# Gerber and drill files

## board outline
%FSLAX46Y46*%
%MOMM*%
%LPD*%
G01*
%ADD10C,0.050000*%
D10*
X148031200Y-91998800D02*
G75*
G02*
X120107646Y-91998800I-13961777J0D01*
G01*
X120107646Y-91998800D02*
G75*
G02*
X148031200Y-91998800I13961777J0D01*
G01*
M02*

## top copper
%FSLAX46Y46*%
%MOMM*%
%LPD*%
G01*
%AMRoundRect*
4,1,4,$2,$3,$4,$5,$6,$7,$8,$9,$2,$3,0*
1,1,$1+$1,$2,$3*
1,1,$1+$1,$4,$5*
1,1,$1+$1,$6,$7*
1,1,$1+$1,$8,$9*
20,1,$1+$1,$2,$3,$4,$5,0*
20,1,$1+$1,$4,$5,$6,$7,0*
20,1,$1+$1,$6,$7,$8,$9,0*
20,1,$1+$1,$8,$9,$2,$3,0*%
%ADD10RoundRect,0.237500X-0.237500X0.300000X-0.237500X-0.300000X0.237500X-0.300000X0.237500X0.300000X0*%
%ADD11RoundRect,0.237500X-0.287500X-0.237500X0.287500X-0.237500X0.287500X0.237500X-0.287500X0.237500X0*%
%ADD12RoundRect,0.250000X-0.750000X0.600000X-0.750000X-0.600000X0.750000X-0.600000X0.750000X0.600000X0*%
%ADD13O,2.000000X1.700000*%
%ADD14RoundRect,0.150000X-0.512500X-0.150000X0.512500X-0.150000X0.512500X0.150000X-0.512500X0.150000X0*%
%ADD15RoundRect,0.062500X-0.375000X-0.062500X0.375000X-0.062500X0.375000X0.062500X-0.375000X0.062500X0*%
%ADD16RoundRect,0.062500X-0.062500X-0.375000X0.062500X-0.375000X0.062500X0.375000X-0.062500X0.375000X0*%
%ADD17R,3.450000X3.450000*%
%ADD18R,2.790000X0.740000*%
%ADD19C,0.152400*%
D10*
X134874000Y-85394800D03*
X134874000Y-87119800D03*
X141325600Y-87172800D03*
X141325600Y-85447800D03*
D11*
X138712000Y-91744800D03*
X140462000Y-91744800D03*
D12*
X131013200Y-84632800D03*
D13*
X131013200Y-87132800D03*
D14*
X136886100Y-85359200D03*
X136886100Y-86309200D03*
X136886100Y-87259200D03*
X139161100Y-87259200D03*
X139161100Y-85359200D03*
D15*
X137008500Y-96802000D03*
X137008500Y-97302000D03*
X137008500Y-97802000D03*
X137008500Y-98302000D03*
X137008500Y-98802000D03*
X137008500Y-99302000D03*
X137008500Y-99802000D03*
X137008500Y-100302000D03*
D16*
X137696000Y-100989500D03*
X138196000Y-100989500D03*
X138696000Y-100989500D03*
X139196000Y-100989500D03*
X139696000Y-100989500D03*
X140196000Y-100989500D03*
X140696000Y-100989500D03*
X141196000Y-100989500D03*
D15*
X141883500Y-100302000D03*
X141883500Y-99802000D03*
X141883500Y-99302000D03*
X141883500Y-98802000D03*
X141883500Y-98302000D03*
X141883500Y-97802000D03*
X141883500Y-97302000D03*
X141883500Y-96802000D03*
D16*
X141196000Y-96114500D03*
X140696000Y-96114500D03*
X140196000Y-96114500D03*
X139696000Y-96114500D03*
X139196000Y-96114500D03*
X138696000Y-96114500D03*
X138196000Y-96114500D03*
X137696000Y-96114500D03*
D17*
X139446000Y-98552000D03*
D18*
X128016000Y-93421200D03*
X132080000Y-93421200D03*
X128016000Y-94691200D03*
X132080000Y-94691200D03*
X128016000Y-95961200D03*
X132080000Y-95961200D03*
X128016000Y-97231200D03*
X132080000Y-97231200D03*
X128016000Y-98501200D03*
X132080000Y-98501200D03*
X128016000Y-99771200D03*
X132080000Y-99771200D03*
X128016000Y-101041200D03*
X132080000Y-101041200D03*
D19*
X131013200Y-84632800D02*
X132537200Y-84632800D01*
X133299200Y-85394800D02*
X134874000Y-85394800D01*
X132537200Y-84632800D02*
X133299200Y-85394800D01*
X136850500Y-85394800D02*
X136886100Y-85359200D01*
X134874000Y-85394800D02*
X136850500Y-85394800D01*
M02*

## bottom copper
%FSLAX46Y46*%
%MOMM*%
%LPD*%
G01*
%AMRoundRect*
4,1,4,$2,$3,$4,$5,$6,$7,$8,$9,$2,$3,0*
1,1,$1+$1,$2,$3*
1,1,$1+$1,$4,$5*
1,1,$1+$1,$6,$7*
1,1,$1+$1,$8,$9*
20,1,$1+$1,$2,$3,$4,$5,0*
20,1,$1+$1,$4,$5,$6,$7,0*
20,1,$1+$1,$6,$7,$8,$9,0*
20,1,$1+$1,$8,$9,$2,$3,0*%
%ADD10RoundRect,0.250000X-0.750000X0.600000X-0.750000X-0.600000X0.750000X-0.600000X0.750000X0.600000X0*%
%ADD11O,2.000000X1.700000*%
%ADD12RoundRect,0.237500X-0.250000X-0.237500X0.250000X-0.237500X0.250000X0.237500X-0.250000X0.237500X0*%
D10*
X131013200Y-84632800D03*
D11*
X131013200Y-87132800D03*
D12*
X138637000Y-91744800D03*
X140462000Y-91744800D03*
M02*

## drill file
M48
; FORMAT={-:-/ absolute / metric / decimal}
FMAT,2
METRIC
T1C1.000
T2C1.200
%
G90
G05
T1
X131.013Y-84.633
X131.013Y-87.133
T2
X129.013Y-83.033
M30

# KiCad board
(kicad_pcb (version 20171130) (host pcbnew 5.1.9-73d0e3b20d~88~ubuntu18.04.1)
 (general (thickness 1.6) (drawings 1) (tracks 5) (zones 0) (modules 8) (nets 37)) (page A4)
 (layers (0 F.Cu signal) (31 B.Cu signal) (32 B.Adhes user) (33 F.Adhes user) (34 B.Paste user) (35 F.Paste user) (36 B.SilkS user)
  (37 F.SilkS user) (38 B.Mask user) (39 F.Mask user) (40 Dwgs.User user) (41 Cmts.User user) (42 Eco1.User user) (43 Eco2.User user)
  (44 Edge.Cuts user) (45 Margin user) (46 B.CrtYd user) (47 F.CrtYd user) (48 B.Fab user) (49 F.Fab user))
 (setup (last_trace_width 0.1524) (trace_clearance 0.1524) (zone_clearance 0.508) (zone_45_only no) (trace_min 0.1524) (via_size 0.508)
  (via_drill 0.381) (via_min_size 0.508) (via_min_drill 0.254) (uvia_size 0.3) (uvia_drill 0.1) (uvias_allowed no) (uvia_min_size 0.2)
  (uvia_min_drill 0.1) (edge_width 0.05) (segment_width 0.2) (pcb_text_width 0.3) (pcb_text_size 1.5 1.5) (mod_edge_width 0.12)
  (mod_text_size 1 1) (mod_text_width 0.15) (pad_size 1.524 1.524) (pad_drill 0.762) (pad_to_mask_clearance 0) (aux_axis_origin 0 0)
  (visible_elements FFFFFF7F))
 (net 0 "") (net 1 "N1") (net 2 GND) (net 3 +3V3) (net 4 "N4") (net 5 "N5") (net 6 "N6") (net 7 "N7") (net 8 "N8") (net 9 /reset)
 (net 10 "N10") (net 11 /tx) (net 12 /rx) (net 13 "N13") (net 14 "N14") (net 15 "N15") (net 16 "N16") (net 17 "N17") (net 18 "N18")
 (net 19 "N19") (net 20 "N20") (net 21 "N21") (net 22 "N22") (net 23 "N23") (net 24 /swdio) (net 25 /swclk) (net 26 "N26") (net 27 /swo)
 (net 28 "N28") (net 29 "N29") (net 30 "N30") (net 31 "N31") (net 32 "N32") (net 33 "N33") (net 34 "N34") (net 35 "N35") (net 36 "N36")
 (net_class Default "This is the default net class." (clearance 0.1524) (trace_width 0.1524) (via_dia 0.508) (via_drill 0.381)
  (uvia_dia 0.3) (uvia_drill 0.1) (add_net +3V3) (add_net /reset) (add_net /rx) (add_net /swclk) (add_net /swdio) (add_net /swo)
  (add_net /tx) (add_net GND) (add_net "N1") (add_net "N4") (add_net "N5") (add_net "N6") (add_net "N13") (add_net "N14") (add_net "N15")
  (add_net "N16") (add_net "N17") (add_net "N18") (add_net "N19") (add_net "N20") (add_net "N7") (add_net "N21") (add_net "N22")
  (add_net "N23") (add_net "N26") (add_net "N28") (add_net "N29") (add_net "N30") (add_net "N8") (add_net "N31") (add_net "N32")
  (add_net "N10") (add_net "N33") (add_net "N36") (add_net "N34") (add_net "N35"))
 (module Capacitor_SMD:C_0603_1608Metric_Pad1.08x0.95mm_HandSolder (layer F.Cu) (at 134.874 86.2573 270)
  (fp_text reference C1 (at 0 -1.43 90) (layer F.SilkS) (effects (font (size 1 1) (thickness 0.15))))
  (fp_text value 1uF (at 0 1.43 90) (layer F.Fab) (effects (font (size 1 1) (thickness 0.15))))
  (pad 1 smd roundrect (at -0.8625 0 270) (size 1.075 0.95) (layers F.Cu F.Paste F.Mask) (roundrect_rratio 0.25) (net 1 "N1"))
  (pad 2 smd roundrect (at 0.8625 0 270) (size 1.075 0.95) (layers F.Cu F.Paste F.Mask) (roundrect_rratio 0.25) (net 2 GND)))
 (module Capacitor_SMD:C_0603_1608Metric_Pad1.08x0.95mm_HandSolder (layer F.Cu) (at 141.3256 86.3103 270)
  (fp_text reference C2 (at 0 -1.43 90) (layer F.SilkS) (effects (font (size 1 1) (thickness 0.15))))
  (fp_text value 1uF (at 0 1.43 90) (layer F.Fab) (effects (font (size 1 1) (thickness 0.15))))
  (pad 2 smd roundrect (at 0.8625 0 270) (size 1.075 0.95) (layers F.Cu F.Paste F.Mask) (roundrect_rratio 0.25) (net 2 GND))
  (pad 1 smd roundrect (at -0.8625 0 270) (size 1.075 0.95) (layers F.Cu F.Paste F.Mask) (roundrect_rratio 0.25) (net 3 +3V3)))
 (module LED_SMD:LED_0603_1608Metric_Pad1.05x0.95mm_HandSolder (layer F.Cu) (at 139.587 91.7448)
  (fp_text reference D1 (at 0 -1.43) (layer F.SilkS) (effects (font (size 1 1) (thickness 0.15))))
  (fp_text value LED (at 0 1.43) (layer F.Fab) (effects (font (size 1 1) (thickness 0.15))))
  (pad 1 smd roundrect (at -0.875 0) (size 1.05 0.95) (layers F.Cu F.Paste F.Mask) (roundrect_rratio 0.25) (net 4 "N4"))
  (pad 2 smd roundrect (at 0.875 0) (size 1.05 0.95) (layers F.Cu F.Paste F.Mask) (roundrect_rratio 0.25) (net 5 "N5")))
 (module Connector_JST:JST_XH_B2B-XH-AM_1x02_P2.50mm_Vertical (layer F.Cu) (at 131.0132 84.6328 270)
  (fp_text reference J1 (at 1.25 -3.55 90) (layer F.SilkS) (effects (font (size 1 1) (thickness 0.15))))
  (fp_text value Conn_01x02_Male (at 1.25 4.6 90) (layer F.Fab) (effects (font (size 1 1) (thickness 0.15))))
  (pad 1 thru_hole roundrect (at 0 0 270) (size 1.7 2) (drill 1) (layers *.Cu *.Mask) (roundrect_rratio 0.147059) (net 1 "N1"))
  (pad 2 thru_hole oval (at 2.5 0 270) (size 1.7 2) (drill 1) (layers *.Cu *.Mask) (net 2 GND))
  (pad "" np_thru_hole circle (at -1.6 2 270) (size 1.2 1.2) (drill 1.2) (layers *.Cu *.Mask)))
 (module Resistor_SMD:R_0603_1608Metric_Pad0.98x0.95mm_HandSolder (layer B.Cu) (at 139.5495 91.7448)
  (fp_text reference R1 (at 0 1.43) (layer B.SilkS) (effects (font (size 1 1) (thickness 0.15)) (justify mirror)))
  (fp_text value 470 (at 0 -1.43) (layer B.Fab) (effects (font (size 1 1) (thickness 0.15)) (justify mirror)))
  (pad 1 smd roundrect (at -0.9125 0) (size 0.975 0.95) (layers B.Cu B.Paste B.Mask) (roundrect_rratio 0.25) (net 3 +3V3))
  (pad 2 smd roundrect (at 0.9125 0) (size 0.975 0.95) (layers B.Cu B.Paste B.Mask) (roundrect_rratio 0.25) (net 5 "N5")))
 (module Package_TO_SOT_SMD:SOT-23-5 (layer F.Cu) (at 138.0236 86.3092)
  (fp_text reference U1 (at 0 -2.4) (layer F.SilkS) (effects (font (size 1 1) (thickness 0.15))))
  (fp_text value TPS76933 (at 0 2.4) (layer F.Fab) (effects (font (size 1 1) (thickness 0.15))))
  (pad 1 smd roundrect (at -1.1375 -0.95) (size 1.325 0.6) (layers F.Cu F.Paste F.Mask) (roundrect_rratio 0.25) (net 1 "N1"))
  (pad 2 smd roundrect (at -1.1375 0) (size 1.325 0.6) (layers F.Cu F.Paste F.Mask) (roundrect_rratio 0.25) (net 2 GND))
  (pad 3 smd roundrect (at -1.1375 0.95) (size 1.325 0.6) (layers F.Cu F.Paste F.Mask) (roundrect_rratio 0.25) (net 2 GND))
  (pad 4 smd roundrect (at 1.1375 0.95) (size 1.325 0.6) (layers F.Cu F.Paste F.Mask) (roundrect_rratio 0.25) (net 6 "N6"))
  (pad 5 smd roundrect (at 1.1375 -0.95) (size 1.325 0.6) (layers F.Cu F.Paste F.Mask) (roundrect_rratio 0.25) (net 3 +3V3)))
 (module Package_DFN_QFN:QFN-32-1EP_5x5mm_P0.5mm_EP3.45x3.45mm (layer F.Cu) (at 139.446 98.552)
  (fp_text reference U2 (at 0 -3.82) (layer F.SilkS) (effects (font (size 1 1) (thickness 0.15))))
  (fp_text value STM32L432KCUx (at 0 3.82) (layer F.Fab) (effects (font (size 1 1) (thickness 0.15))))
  (pad 1 smd roundrect (at -2.4375 -1.75) (size 0.875 0.25) (layers F.Cu F.Paste F.Mask) (roundrect_rratio 0.25) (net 3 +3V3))
  (pad 2 smd roundrect (at -2.4375 -1.25) (size 0.875 0.25) (layers F.Cu F.Paste F.Mask) (roundrect_rratio 0.25) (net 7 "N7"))
  (pad 3 smd roundrect (at -2.4375 -0.75) (size 0.875 0.25) (layers F.Cu F.Paste F.Mask) (roundrect_rratio 0.25) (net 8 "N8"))
  (pad 4 smd roundrect (at -2.4375 -0.25) (size 0.875 0.25) (layers F.Cu F.Paste F.Mask) (roundrect_rratio 0.25) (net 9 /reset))
  (pad 5 smd roundrect (at -2.4375 0.25) (size 0.875 0.25) (layers F.Cu F.Paste F.Mask) (roundrect_rratio 0.25) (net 3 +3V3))
  (pad 6 smd roundrect (at -2.4375 0.75) (size 0.875 0.25) (layers F.Cu F.Paste F.Mask) (roundrect_rratio 0.25) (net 4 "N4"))
  (pad 7 smd roundrect (at -2.4375 1.25) (size 0.875 0.25) (layers F.Cu F.Paste F.Mask) (roundrect_rratio 0.25) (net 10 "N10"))
  (pad 8 smd roundrect (at -2.4375 1.75) (size 0.875 0.25) (layers F.Cu F.Paste F.Mask) (roundrect_rratio 0.25) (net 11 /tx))
  (pad 9 smd roundrect (at -1.75 2.4375) (size 0.25 0.875) (layers F.Cu F.Paste F.Mask) (roundrect_rratio 0.25) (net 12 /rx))
  (pad 10 smd roundrect (at -1.25 2.4375) (size 0.25 0.875) (layers F.Cu F.Paste F.Mask) (roundrect_rratio 0.25) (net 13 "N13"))
  (pad 11 smd roundrect (at -0.75 2.4375) (size 0.25 0.875) (layers F.Cu F.Paste F.Mask) (roundrect_rratio 0.25) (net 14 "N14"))
  (pad 12 smd roundrect (at -0.25 2.4375) (size 0.25 0.875) (layers F.Cu F.Paste F.Mask) (roundrect_rratio 0.25) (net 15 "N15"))
  (pad 13 smd roundrect (at 0.25 2.4375) (size 0.25 0.875) (layers F.Cu F.Paste F.Mask) (roundrect_rratio 0.25) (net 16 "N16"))
  (pad 14 smd roundrect (at 0.75 2.4375) (size 0.25 0.875) (layers F.Cu F.Paste F.Mask) (roundrect_rratio 0.25) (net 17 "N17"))
  (pad 15 smd roundrect (at 1.25 2.4375) (size 0.25 0.875) (layers F.Cu F.Paste F.Mask) (roundrect_rratio 0.25) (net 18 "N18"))
  (pad 16 smd roundrect (at 1.75 2.4375) (size 0.25 0.875) (layers F.Cu F.Paste F.Mask) (roundrect_rratio 0.25) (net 2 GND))
  (pad 17 smd roundrect (at 2.4375 1.75) (size 0.875 0.25) (layers F.Cu F.Paste F.Mask) (roundrect_rratio 0.25) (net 3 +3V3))
  (pad 18 smd roundrect (at 2.4375 1.25) (size 0.875 0.25) (layers F.Cu F.Paste F.Mask) (roundrect_rratio 0.25) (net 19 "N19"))
  (pad 19 smd roundrect (at 2.4375 0.75) (size 0.875 0.25) (layers F.Cu F.Paste F.Mask) (roundrect_rratio 0.25) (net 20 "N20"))
  (pad 20 smd roundrect (at 2.4375 0.25) (size 0.875 0.25) (layers F.Cu F.Paste F.Mask) (roundrect_rratio 0.25) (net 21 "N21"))
  (pad 21 smd roundrect (at 2.4375 -0.25) (size 0.875 0.25) (layers F.Cu F.Paste F.Mask) (roundrect_rratio 0.25) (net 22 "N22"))
  (pad 22 smd roundrect (at 2.4375 -0.75) (size 0.875 0.25) (layers F.Cu F.Paste F.Mask) (roundrect_rratio 0.25) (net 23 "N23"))
  (pad 23 smd roundrect (at 2.4375 -1.25) (size 0.875 0.25) (layers F.Cu F.Paste F.Mask) (roundrect_rratio 0.25) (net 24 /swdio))
  (pad 24 smd roundrect (at 2.4375 -1.75) (size 0.875 0.25) (layers F.Cu F.Paste F.Mask) (roundrect_rratio 0.25) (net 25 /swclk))
  (pad 25 smd roundrect (at 1.75 -2.4375) (size 0.25 0.875) (layers F.Cu F.Paste F.Mask) (roundrect_rratio 0.25) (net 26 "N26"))
  (pad 26 smd roundrect (at 1.25 -2.4375) (size 0.25 0.875) (layers F.Cu F.Paste F.Mask) (roundrect_rratio 0.25) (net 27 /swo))
  (pad 27 smd roundrect (at 0.75 -2.4375) (size 0.25 0.875) (layers F.Cu F.Paste F.Mask) (roundrect_rratio 0.25) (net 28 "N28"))
  (pad 28 smd roundrect (at 0.25 -2.4375) (size 0.25 0.875) (layers F.Cu F.Paste F.Mask) (roundrect_rratio 0.25) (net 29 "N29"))
  (pad 29 smd roundrect (at -0.25 -2.4375) (size 0.25 0.875) (layers F.Cu F.Paste F.Mask) (roundrect_rratio 0.25) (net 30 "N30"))
  (pad 30 smd roundrect (at -0.75 -2.4375) (size 0.25 0.875) (layers F.Cu F.Paste F.Mask) (roundrect_rratio 0.25) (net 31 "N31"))
  (pad 31 smd roundrect (at -1.25 -2.4375) (size 0.25 0.875) (layers F.Cu F.Paste F.Mask) (roundrect_rratio 0.25) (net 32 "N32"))
  (pad 32 smd roundrect (at -1.75 -2.4375) (size 0.25 0.875) (layers F.Cu F.Paste F.Mask) (roundrect_rratio 0.25) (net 2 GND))
  (pad 33 smd rect (at 0 0) (size 3.45 3.45) (layers F.Cu F.Mask) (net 2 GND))
  (pad "" smd roundrect (at -1.15 -1.15) (size 0.93 0.93) (layers F.Paste) (roundrect_rratio 0.25))
  (pad "" smd roundrect (at -1.15 0) (size 0.93 0.93) (layers F.Paste) (roundrect_rratio 0.25))
  (pad "" smd roundrect (at -1.15 1.15) (size 0.93 0.93) (layers F.Paste) (roundrect_rratio 0.25))
  (pad "" smd roundrect (at 0 -1.15) (size 0.93 0.93) (layers F.Paste) (roundrect_rratio 0.25))
  (pad "" smd roundrect (at 0 0) (size 0.93 0.93) (layers F.Paste) (roundrect_rratio 0.25))
  (pad "" smd roundrect (at 0 1.15) (size 0.93 0.93) (layers F.Paste) (roundrect_rratio 0.25))
  (pad "" smd roundrect (at 1.15 -1.15) (size 0.93 0.93) (layers F.Paste) (roundrect_rratio 0.25))
  (pad "" smd roundrect (at 1.15 0) (size 0.93 0.93) (layers F.Paste) (roundrect_rratio 0.25))
  (pad "" smd roundrect (at 1.15 1.15) (size 0.93 0.93) (layers F.Paste) (roundrect_rratio 0.25)))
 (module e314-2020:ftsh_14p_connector (layer F.Cu) (at 130.048 97.2312 270)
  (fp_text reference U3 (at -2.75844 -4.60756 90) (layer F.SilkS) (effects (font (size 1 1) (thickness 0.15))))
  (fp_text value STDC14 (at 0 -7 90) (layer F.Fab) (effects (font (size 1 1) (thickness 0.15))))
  (pad 1 smd rect (at -3.81 2.032 270) (size 0.74 2.79) (layers F.Cu F.Paste F.Mask) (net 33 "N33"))
  (pad 2 smd rect (at -3.81 -2.032 270) (size 0.74 2.79) (layers F.Cu F.Paste F.Mask) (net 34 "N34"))
  (pad 3 smd rect (at -2.54 2.032 270) (size 0.74 2.79) (layers F.Cu F.Paste F.Mask) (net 3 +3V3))
  (pad 4 smd rect (at -2.54 -2.032 270) (size 0.74 2.79) (layers F.Cu F.Paste F.Mask) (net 24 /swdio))
  (pad 5 smd rect (at -1.27 2.032 270) (size 0.74 2.79) (layers F.Cu F.Paste F.Mask) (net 2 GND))
  (pad 6 smd rect (at -1.27 -2.032 270) (size 0.74 2.79) (layers F.Cu F.Paste F.Mask) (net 25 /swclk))
  (pad 7 smd rect (at 0 2.032 270) (size 0.74 2.79) (layers F.Cu F.Paste F.Mask) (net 2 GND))
  (pad 8 smd rect (at 0 -2.032 270) (size 0.74 2.79) (layers F.Cu F.Paste F.Mask) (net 27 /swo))
  (pad 9 smd rect (at 1.27 2.032 270) (size 0.74 2.79) (layers F.Cu F.Paste F.Mask) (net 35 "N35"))
  (pad 10 smd rect (at 1.27 -2.032 270) (size 0.74 2.79) (layers F.Cu F.Paste F.Mask) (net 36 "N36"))
  (pad 11 smd rect (at 2.54 2.032 270) (size 0.74 2.79) (layers F.Cu F.Paste F.Mask) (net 2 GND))
  (pad 12 smd rect (at 2.54 -2.032 270) (size 0.74 2.79) (layers F.Cu F.Paste F.Mask) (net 9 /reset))
  (pad 13 smd rect (at 3.81 2.032 270) (size 0.74 2.79) (layers F.Cu F.Paste F.Mask) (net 11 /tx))
  (pad 14 smd rect (at 3.81 -2.032 270) (size 0.74 2.79) (layers F.Cu F.Paste F.Mask) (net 12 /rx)))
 (gr_circle (center 134.069423 91.9988) (end 121.064623 86.9188) (layer Edge.Cuts) (width 0.05))
 (segment (start 131.0132 84.6328) (end 132.5372 84.6328) (width 0.1524) (layer F.Cu) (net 1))
 (segment (start 133.2992 85.3948) (end 134.874 85.3948) (width 0.1524) (layer F.Cu) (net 1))
 (segment (start 132.5372 84.6328) (end 133.2992 85.3948) (width 0.1524) (layer F.Cu) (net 1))
 (segment (start 136.8505 85.3948) (end 136.8861 85.3592) (width 0.1524) (layer F.Cu) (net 1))
 (segment (start 134.874 85.3948) (end 136.8505 85.3948) (width 0.1524) (layer F.Cu) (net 1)))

